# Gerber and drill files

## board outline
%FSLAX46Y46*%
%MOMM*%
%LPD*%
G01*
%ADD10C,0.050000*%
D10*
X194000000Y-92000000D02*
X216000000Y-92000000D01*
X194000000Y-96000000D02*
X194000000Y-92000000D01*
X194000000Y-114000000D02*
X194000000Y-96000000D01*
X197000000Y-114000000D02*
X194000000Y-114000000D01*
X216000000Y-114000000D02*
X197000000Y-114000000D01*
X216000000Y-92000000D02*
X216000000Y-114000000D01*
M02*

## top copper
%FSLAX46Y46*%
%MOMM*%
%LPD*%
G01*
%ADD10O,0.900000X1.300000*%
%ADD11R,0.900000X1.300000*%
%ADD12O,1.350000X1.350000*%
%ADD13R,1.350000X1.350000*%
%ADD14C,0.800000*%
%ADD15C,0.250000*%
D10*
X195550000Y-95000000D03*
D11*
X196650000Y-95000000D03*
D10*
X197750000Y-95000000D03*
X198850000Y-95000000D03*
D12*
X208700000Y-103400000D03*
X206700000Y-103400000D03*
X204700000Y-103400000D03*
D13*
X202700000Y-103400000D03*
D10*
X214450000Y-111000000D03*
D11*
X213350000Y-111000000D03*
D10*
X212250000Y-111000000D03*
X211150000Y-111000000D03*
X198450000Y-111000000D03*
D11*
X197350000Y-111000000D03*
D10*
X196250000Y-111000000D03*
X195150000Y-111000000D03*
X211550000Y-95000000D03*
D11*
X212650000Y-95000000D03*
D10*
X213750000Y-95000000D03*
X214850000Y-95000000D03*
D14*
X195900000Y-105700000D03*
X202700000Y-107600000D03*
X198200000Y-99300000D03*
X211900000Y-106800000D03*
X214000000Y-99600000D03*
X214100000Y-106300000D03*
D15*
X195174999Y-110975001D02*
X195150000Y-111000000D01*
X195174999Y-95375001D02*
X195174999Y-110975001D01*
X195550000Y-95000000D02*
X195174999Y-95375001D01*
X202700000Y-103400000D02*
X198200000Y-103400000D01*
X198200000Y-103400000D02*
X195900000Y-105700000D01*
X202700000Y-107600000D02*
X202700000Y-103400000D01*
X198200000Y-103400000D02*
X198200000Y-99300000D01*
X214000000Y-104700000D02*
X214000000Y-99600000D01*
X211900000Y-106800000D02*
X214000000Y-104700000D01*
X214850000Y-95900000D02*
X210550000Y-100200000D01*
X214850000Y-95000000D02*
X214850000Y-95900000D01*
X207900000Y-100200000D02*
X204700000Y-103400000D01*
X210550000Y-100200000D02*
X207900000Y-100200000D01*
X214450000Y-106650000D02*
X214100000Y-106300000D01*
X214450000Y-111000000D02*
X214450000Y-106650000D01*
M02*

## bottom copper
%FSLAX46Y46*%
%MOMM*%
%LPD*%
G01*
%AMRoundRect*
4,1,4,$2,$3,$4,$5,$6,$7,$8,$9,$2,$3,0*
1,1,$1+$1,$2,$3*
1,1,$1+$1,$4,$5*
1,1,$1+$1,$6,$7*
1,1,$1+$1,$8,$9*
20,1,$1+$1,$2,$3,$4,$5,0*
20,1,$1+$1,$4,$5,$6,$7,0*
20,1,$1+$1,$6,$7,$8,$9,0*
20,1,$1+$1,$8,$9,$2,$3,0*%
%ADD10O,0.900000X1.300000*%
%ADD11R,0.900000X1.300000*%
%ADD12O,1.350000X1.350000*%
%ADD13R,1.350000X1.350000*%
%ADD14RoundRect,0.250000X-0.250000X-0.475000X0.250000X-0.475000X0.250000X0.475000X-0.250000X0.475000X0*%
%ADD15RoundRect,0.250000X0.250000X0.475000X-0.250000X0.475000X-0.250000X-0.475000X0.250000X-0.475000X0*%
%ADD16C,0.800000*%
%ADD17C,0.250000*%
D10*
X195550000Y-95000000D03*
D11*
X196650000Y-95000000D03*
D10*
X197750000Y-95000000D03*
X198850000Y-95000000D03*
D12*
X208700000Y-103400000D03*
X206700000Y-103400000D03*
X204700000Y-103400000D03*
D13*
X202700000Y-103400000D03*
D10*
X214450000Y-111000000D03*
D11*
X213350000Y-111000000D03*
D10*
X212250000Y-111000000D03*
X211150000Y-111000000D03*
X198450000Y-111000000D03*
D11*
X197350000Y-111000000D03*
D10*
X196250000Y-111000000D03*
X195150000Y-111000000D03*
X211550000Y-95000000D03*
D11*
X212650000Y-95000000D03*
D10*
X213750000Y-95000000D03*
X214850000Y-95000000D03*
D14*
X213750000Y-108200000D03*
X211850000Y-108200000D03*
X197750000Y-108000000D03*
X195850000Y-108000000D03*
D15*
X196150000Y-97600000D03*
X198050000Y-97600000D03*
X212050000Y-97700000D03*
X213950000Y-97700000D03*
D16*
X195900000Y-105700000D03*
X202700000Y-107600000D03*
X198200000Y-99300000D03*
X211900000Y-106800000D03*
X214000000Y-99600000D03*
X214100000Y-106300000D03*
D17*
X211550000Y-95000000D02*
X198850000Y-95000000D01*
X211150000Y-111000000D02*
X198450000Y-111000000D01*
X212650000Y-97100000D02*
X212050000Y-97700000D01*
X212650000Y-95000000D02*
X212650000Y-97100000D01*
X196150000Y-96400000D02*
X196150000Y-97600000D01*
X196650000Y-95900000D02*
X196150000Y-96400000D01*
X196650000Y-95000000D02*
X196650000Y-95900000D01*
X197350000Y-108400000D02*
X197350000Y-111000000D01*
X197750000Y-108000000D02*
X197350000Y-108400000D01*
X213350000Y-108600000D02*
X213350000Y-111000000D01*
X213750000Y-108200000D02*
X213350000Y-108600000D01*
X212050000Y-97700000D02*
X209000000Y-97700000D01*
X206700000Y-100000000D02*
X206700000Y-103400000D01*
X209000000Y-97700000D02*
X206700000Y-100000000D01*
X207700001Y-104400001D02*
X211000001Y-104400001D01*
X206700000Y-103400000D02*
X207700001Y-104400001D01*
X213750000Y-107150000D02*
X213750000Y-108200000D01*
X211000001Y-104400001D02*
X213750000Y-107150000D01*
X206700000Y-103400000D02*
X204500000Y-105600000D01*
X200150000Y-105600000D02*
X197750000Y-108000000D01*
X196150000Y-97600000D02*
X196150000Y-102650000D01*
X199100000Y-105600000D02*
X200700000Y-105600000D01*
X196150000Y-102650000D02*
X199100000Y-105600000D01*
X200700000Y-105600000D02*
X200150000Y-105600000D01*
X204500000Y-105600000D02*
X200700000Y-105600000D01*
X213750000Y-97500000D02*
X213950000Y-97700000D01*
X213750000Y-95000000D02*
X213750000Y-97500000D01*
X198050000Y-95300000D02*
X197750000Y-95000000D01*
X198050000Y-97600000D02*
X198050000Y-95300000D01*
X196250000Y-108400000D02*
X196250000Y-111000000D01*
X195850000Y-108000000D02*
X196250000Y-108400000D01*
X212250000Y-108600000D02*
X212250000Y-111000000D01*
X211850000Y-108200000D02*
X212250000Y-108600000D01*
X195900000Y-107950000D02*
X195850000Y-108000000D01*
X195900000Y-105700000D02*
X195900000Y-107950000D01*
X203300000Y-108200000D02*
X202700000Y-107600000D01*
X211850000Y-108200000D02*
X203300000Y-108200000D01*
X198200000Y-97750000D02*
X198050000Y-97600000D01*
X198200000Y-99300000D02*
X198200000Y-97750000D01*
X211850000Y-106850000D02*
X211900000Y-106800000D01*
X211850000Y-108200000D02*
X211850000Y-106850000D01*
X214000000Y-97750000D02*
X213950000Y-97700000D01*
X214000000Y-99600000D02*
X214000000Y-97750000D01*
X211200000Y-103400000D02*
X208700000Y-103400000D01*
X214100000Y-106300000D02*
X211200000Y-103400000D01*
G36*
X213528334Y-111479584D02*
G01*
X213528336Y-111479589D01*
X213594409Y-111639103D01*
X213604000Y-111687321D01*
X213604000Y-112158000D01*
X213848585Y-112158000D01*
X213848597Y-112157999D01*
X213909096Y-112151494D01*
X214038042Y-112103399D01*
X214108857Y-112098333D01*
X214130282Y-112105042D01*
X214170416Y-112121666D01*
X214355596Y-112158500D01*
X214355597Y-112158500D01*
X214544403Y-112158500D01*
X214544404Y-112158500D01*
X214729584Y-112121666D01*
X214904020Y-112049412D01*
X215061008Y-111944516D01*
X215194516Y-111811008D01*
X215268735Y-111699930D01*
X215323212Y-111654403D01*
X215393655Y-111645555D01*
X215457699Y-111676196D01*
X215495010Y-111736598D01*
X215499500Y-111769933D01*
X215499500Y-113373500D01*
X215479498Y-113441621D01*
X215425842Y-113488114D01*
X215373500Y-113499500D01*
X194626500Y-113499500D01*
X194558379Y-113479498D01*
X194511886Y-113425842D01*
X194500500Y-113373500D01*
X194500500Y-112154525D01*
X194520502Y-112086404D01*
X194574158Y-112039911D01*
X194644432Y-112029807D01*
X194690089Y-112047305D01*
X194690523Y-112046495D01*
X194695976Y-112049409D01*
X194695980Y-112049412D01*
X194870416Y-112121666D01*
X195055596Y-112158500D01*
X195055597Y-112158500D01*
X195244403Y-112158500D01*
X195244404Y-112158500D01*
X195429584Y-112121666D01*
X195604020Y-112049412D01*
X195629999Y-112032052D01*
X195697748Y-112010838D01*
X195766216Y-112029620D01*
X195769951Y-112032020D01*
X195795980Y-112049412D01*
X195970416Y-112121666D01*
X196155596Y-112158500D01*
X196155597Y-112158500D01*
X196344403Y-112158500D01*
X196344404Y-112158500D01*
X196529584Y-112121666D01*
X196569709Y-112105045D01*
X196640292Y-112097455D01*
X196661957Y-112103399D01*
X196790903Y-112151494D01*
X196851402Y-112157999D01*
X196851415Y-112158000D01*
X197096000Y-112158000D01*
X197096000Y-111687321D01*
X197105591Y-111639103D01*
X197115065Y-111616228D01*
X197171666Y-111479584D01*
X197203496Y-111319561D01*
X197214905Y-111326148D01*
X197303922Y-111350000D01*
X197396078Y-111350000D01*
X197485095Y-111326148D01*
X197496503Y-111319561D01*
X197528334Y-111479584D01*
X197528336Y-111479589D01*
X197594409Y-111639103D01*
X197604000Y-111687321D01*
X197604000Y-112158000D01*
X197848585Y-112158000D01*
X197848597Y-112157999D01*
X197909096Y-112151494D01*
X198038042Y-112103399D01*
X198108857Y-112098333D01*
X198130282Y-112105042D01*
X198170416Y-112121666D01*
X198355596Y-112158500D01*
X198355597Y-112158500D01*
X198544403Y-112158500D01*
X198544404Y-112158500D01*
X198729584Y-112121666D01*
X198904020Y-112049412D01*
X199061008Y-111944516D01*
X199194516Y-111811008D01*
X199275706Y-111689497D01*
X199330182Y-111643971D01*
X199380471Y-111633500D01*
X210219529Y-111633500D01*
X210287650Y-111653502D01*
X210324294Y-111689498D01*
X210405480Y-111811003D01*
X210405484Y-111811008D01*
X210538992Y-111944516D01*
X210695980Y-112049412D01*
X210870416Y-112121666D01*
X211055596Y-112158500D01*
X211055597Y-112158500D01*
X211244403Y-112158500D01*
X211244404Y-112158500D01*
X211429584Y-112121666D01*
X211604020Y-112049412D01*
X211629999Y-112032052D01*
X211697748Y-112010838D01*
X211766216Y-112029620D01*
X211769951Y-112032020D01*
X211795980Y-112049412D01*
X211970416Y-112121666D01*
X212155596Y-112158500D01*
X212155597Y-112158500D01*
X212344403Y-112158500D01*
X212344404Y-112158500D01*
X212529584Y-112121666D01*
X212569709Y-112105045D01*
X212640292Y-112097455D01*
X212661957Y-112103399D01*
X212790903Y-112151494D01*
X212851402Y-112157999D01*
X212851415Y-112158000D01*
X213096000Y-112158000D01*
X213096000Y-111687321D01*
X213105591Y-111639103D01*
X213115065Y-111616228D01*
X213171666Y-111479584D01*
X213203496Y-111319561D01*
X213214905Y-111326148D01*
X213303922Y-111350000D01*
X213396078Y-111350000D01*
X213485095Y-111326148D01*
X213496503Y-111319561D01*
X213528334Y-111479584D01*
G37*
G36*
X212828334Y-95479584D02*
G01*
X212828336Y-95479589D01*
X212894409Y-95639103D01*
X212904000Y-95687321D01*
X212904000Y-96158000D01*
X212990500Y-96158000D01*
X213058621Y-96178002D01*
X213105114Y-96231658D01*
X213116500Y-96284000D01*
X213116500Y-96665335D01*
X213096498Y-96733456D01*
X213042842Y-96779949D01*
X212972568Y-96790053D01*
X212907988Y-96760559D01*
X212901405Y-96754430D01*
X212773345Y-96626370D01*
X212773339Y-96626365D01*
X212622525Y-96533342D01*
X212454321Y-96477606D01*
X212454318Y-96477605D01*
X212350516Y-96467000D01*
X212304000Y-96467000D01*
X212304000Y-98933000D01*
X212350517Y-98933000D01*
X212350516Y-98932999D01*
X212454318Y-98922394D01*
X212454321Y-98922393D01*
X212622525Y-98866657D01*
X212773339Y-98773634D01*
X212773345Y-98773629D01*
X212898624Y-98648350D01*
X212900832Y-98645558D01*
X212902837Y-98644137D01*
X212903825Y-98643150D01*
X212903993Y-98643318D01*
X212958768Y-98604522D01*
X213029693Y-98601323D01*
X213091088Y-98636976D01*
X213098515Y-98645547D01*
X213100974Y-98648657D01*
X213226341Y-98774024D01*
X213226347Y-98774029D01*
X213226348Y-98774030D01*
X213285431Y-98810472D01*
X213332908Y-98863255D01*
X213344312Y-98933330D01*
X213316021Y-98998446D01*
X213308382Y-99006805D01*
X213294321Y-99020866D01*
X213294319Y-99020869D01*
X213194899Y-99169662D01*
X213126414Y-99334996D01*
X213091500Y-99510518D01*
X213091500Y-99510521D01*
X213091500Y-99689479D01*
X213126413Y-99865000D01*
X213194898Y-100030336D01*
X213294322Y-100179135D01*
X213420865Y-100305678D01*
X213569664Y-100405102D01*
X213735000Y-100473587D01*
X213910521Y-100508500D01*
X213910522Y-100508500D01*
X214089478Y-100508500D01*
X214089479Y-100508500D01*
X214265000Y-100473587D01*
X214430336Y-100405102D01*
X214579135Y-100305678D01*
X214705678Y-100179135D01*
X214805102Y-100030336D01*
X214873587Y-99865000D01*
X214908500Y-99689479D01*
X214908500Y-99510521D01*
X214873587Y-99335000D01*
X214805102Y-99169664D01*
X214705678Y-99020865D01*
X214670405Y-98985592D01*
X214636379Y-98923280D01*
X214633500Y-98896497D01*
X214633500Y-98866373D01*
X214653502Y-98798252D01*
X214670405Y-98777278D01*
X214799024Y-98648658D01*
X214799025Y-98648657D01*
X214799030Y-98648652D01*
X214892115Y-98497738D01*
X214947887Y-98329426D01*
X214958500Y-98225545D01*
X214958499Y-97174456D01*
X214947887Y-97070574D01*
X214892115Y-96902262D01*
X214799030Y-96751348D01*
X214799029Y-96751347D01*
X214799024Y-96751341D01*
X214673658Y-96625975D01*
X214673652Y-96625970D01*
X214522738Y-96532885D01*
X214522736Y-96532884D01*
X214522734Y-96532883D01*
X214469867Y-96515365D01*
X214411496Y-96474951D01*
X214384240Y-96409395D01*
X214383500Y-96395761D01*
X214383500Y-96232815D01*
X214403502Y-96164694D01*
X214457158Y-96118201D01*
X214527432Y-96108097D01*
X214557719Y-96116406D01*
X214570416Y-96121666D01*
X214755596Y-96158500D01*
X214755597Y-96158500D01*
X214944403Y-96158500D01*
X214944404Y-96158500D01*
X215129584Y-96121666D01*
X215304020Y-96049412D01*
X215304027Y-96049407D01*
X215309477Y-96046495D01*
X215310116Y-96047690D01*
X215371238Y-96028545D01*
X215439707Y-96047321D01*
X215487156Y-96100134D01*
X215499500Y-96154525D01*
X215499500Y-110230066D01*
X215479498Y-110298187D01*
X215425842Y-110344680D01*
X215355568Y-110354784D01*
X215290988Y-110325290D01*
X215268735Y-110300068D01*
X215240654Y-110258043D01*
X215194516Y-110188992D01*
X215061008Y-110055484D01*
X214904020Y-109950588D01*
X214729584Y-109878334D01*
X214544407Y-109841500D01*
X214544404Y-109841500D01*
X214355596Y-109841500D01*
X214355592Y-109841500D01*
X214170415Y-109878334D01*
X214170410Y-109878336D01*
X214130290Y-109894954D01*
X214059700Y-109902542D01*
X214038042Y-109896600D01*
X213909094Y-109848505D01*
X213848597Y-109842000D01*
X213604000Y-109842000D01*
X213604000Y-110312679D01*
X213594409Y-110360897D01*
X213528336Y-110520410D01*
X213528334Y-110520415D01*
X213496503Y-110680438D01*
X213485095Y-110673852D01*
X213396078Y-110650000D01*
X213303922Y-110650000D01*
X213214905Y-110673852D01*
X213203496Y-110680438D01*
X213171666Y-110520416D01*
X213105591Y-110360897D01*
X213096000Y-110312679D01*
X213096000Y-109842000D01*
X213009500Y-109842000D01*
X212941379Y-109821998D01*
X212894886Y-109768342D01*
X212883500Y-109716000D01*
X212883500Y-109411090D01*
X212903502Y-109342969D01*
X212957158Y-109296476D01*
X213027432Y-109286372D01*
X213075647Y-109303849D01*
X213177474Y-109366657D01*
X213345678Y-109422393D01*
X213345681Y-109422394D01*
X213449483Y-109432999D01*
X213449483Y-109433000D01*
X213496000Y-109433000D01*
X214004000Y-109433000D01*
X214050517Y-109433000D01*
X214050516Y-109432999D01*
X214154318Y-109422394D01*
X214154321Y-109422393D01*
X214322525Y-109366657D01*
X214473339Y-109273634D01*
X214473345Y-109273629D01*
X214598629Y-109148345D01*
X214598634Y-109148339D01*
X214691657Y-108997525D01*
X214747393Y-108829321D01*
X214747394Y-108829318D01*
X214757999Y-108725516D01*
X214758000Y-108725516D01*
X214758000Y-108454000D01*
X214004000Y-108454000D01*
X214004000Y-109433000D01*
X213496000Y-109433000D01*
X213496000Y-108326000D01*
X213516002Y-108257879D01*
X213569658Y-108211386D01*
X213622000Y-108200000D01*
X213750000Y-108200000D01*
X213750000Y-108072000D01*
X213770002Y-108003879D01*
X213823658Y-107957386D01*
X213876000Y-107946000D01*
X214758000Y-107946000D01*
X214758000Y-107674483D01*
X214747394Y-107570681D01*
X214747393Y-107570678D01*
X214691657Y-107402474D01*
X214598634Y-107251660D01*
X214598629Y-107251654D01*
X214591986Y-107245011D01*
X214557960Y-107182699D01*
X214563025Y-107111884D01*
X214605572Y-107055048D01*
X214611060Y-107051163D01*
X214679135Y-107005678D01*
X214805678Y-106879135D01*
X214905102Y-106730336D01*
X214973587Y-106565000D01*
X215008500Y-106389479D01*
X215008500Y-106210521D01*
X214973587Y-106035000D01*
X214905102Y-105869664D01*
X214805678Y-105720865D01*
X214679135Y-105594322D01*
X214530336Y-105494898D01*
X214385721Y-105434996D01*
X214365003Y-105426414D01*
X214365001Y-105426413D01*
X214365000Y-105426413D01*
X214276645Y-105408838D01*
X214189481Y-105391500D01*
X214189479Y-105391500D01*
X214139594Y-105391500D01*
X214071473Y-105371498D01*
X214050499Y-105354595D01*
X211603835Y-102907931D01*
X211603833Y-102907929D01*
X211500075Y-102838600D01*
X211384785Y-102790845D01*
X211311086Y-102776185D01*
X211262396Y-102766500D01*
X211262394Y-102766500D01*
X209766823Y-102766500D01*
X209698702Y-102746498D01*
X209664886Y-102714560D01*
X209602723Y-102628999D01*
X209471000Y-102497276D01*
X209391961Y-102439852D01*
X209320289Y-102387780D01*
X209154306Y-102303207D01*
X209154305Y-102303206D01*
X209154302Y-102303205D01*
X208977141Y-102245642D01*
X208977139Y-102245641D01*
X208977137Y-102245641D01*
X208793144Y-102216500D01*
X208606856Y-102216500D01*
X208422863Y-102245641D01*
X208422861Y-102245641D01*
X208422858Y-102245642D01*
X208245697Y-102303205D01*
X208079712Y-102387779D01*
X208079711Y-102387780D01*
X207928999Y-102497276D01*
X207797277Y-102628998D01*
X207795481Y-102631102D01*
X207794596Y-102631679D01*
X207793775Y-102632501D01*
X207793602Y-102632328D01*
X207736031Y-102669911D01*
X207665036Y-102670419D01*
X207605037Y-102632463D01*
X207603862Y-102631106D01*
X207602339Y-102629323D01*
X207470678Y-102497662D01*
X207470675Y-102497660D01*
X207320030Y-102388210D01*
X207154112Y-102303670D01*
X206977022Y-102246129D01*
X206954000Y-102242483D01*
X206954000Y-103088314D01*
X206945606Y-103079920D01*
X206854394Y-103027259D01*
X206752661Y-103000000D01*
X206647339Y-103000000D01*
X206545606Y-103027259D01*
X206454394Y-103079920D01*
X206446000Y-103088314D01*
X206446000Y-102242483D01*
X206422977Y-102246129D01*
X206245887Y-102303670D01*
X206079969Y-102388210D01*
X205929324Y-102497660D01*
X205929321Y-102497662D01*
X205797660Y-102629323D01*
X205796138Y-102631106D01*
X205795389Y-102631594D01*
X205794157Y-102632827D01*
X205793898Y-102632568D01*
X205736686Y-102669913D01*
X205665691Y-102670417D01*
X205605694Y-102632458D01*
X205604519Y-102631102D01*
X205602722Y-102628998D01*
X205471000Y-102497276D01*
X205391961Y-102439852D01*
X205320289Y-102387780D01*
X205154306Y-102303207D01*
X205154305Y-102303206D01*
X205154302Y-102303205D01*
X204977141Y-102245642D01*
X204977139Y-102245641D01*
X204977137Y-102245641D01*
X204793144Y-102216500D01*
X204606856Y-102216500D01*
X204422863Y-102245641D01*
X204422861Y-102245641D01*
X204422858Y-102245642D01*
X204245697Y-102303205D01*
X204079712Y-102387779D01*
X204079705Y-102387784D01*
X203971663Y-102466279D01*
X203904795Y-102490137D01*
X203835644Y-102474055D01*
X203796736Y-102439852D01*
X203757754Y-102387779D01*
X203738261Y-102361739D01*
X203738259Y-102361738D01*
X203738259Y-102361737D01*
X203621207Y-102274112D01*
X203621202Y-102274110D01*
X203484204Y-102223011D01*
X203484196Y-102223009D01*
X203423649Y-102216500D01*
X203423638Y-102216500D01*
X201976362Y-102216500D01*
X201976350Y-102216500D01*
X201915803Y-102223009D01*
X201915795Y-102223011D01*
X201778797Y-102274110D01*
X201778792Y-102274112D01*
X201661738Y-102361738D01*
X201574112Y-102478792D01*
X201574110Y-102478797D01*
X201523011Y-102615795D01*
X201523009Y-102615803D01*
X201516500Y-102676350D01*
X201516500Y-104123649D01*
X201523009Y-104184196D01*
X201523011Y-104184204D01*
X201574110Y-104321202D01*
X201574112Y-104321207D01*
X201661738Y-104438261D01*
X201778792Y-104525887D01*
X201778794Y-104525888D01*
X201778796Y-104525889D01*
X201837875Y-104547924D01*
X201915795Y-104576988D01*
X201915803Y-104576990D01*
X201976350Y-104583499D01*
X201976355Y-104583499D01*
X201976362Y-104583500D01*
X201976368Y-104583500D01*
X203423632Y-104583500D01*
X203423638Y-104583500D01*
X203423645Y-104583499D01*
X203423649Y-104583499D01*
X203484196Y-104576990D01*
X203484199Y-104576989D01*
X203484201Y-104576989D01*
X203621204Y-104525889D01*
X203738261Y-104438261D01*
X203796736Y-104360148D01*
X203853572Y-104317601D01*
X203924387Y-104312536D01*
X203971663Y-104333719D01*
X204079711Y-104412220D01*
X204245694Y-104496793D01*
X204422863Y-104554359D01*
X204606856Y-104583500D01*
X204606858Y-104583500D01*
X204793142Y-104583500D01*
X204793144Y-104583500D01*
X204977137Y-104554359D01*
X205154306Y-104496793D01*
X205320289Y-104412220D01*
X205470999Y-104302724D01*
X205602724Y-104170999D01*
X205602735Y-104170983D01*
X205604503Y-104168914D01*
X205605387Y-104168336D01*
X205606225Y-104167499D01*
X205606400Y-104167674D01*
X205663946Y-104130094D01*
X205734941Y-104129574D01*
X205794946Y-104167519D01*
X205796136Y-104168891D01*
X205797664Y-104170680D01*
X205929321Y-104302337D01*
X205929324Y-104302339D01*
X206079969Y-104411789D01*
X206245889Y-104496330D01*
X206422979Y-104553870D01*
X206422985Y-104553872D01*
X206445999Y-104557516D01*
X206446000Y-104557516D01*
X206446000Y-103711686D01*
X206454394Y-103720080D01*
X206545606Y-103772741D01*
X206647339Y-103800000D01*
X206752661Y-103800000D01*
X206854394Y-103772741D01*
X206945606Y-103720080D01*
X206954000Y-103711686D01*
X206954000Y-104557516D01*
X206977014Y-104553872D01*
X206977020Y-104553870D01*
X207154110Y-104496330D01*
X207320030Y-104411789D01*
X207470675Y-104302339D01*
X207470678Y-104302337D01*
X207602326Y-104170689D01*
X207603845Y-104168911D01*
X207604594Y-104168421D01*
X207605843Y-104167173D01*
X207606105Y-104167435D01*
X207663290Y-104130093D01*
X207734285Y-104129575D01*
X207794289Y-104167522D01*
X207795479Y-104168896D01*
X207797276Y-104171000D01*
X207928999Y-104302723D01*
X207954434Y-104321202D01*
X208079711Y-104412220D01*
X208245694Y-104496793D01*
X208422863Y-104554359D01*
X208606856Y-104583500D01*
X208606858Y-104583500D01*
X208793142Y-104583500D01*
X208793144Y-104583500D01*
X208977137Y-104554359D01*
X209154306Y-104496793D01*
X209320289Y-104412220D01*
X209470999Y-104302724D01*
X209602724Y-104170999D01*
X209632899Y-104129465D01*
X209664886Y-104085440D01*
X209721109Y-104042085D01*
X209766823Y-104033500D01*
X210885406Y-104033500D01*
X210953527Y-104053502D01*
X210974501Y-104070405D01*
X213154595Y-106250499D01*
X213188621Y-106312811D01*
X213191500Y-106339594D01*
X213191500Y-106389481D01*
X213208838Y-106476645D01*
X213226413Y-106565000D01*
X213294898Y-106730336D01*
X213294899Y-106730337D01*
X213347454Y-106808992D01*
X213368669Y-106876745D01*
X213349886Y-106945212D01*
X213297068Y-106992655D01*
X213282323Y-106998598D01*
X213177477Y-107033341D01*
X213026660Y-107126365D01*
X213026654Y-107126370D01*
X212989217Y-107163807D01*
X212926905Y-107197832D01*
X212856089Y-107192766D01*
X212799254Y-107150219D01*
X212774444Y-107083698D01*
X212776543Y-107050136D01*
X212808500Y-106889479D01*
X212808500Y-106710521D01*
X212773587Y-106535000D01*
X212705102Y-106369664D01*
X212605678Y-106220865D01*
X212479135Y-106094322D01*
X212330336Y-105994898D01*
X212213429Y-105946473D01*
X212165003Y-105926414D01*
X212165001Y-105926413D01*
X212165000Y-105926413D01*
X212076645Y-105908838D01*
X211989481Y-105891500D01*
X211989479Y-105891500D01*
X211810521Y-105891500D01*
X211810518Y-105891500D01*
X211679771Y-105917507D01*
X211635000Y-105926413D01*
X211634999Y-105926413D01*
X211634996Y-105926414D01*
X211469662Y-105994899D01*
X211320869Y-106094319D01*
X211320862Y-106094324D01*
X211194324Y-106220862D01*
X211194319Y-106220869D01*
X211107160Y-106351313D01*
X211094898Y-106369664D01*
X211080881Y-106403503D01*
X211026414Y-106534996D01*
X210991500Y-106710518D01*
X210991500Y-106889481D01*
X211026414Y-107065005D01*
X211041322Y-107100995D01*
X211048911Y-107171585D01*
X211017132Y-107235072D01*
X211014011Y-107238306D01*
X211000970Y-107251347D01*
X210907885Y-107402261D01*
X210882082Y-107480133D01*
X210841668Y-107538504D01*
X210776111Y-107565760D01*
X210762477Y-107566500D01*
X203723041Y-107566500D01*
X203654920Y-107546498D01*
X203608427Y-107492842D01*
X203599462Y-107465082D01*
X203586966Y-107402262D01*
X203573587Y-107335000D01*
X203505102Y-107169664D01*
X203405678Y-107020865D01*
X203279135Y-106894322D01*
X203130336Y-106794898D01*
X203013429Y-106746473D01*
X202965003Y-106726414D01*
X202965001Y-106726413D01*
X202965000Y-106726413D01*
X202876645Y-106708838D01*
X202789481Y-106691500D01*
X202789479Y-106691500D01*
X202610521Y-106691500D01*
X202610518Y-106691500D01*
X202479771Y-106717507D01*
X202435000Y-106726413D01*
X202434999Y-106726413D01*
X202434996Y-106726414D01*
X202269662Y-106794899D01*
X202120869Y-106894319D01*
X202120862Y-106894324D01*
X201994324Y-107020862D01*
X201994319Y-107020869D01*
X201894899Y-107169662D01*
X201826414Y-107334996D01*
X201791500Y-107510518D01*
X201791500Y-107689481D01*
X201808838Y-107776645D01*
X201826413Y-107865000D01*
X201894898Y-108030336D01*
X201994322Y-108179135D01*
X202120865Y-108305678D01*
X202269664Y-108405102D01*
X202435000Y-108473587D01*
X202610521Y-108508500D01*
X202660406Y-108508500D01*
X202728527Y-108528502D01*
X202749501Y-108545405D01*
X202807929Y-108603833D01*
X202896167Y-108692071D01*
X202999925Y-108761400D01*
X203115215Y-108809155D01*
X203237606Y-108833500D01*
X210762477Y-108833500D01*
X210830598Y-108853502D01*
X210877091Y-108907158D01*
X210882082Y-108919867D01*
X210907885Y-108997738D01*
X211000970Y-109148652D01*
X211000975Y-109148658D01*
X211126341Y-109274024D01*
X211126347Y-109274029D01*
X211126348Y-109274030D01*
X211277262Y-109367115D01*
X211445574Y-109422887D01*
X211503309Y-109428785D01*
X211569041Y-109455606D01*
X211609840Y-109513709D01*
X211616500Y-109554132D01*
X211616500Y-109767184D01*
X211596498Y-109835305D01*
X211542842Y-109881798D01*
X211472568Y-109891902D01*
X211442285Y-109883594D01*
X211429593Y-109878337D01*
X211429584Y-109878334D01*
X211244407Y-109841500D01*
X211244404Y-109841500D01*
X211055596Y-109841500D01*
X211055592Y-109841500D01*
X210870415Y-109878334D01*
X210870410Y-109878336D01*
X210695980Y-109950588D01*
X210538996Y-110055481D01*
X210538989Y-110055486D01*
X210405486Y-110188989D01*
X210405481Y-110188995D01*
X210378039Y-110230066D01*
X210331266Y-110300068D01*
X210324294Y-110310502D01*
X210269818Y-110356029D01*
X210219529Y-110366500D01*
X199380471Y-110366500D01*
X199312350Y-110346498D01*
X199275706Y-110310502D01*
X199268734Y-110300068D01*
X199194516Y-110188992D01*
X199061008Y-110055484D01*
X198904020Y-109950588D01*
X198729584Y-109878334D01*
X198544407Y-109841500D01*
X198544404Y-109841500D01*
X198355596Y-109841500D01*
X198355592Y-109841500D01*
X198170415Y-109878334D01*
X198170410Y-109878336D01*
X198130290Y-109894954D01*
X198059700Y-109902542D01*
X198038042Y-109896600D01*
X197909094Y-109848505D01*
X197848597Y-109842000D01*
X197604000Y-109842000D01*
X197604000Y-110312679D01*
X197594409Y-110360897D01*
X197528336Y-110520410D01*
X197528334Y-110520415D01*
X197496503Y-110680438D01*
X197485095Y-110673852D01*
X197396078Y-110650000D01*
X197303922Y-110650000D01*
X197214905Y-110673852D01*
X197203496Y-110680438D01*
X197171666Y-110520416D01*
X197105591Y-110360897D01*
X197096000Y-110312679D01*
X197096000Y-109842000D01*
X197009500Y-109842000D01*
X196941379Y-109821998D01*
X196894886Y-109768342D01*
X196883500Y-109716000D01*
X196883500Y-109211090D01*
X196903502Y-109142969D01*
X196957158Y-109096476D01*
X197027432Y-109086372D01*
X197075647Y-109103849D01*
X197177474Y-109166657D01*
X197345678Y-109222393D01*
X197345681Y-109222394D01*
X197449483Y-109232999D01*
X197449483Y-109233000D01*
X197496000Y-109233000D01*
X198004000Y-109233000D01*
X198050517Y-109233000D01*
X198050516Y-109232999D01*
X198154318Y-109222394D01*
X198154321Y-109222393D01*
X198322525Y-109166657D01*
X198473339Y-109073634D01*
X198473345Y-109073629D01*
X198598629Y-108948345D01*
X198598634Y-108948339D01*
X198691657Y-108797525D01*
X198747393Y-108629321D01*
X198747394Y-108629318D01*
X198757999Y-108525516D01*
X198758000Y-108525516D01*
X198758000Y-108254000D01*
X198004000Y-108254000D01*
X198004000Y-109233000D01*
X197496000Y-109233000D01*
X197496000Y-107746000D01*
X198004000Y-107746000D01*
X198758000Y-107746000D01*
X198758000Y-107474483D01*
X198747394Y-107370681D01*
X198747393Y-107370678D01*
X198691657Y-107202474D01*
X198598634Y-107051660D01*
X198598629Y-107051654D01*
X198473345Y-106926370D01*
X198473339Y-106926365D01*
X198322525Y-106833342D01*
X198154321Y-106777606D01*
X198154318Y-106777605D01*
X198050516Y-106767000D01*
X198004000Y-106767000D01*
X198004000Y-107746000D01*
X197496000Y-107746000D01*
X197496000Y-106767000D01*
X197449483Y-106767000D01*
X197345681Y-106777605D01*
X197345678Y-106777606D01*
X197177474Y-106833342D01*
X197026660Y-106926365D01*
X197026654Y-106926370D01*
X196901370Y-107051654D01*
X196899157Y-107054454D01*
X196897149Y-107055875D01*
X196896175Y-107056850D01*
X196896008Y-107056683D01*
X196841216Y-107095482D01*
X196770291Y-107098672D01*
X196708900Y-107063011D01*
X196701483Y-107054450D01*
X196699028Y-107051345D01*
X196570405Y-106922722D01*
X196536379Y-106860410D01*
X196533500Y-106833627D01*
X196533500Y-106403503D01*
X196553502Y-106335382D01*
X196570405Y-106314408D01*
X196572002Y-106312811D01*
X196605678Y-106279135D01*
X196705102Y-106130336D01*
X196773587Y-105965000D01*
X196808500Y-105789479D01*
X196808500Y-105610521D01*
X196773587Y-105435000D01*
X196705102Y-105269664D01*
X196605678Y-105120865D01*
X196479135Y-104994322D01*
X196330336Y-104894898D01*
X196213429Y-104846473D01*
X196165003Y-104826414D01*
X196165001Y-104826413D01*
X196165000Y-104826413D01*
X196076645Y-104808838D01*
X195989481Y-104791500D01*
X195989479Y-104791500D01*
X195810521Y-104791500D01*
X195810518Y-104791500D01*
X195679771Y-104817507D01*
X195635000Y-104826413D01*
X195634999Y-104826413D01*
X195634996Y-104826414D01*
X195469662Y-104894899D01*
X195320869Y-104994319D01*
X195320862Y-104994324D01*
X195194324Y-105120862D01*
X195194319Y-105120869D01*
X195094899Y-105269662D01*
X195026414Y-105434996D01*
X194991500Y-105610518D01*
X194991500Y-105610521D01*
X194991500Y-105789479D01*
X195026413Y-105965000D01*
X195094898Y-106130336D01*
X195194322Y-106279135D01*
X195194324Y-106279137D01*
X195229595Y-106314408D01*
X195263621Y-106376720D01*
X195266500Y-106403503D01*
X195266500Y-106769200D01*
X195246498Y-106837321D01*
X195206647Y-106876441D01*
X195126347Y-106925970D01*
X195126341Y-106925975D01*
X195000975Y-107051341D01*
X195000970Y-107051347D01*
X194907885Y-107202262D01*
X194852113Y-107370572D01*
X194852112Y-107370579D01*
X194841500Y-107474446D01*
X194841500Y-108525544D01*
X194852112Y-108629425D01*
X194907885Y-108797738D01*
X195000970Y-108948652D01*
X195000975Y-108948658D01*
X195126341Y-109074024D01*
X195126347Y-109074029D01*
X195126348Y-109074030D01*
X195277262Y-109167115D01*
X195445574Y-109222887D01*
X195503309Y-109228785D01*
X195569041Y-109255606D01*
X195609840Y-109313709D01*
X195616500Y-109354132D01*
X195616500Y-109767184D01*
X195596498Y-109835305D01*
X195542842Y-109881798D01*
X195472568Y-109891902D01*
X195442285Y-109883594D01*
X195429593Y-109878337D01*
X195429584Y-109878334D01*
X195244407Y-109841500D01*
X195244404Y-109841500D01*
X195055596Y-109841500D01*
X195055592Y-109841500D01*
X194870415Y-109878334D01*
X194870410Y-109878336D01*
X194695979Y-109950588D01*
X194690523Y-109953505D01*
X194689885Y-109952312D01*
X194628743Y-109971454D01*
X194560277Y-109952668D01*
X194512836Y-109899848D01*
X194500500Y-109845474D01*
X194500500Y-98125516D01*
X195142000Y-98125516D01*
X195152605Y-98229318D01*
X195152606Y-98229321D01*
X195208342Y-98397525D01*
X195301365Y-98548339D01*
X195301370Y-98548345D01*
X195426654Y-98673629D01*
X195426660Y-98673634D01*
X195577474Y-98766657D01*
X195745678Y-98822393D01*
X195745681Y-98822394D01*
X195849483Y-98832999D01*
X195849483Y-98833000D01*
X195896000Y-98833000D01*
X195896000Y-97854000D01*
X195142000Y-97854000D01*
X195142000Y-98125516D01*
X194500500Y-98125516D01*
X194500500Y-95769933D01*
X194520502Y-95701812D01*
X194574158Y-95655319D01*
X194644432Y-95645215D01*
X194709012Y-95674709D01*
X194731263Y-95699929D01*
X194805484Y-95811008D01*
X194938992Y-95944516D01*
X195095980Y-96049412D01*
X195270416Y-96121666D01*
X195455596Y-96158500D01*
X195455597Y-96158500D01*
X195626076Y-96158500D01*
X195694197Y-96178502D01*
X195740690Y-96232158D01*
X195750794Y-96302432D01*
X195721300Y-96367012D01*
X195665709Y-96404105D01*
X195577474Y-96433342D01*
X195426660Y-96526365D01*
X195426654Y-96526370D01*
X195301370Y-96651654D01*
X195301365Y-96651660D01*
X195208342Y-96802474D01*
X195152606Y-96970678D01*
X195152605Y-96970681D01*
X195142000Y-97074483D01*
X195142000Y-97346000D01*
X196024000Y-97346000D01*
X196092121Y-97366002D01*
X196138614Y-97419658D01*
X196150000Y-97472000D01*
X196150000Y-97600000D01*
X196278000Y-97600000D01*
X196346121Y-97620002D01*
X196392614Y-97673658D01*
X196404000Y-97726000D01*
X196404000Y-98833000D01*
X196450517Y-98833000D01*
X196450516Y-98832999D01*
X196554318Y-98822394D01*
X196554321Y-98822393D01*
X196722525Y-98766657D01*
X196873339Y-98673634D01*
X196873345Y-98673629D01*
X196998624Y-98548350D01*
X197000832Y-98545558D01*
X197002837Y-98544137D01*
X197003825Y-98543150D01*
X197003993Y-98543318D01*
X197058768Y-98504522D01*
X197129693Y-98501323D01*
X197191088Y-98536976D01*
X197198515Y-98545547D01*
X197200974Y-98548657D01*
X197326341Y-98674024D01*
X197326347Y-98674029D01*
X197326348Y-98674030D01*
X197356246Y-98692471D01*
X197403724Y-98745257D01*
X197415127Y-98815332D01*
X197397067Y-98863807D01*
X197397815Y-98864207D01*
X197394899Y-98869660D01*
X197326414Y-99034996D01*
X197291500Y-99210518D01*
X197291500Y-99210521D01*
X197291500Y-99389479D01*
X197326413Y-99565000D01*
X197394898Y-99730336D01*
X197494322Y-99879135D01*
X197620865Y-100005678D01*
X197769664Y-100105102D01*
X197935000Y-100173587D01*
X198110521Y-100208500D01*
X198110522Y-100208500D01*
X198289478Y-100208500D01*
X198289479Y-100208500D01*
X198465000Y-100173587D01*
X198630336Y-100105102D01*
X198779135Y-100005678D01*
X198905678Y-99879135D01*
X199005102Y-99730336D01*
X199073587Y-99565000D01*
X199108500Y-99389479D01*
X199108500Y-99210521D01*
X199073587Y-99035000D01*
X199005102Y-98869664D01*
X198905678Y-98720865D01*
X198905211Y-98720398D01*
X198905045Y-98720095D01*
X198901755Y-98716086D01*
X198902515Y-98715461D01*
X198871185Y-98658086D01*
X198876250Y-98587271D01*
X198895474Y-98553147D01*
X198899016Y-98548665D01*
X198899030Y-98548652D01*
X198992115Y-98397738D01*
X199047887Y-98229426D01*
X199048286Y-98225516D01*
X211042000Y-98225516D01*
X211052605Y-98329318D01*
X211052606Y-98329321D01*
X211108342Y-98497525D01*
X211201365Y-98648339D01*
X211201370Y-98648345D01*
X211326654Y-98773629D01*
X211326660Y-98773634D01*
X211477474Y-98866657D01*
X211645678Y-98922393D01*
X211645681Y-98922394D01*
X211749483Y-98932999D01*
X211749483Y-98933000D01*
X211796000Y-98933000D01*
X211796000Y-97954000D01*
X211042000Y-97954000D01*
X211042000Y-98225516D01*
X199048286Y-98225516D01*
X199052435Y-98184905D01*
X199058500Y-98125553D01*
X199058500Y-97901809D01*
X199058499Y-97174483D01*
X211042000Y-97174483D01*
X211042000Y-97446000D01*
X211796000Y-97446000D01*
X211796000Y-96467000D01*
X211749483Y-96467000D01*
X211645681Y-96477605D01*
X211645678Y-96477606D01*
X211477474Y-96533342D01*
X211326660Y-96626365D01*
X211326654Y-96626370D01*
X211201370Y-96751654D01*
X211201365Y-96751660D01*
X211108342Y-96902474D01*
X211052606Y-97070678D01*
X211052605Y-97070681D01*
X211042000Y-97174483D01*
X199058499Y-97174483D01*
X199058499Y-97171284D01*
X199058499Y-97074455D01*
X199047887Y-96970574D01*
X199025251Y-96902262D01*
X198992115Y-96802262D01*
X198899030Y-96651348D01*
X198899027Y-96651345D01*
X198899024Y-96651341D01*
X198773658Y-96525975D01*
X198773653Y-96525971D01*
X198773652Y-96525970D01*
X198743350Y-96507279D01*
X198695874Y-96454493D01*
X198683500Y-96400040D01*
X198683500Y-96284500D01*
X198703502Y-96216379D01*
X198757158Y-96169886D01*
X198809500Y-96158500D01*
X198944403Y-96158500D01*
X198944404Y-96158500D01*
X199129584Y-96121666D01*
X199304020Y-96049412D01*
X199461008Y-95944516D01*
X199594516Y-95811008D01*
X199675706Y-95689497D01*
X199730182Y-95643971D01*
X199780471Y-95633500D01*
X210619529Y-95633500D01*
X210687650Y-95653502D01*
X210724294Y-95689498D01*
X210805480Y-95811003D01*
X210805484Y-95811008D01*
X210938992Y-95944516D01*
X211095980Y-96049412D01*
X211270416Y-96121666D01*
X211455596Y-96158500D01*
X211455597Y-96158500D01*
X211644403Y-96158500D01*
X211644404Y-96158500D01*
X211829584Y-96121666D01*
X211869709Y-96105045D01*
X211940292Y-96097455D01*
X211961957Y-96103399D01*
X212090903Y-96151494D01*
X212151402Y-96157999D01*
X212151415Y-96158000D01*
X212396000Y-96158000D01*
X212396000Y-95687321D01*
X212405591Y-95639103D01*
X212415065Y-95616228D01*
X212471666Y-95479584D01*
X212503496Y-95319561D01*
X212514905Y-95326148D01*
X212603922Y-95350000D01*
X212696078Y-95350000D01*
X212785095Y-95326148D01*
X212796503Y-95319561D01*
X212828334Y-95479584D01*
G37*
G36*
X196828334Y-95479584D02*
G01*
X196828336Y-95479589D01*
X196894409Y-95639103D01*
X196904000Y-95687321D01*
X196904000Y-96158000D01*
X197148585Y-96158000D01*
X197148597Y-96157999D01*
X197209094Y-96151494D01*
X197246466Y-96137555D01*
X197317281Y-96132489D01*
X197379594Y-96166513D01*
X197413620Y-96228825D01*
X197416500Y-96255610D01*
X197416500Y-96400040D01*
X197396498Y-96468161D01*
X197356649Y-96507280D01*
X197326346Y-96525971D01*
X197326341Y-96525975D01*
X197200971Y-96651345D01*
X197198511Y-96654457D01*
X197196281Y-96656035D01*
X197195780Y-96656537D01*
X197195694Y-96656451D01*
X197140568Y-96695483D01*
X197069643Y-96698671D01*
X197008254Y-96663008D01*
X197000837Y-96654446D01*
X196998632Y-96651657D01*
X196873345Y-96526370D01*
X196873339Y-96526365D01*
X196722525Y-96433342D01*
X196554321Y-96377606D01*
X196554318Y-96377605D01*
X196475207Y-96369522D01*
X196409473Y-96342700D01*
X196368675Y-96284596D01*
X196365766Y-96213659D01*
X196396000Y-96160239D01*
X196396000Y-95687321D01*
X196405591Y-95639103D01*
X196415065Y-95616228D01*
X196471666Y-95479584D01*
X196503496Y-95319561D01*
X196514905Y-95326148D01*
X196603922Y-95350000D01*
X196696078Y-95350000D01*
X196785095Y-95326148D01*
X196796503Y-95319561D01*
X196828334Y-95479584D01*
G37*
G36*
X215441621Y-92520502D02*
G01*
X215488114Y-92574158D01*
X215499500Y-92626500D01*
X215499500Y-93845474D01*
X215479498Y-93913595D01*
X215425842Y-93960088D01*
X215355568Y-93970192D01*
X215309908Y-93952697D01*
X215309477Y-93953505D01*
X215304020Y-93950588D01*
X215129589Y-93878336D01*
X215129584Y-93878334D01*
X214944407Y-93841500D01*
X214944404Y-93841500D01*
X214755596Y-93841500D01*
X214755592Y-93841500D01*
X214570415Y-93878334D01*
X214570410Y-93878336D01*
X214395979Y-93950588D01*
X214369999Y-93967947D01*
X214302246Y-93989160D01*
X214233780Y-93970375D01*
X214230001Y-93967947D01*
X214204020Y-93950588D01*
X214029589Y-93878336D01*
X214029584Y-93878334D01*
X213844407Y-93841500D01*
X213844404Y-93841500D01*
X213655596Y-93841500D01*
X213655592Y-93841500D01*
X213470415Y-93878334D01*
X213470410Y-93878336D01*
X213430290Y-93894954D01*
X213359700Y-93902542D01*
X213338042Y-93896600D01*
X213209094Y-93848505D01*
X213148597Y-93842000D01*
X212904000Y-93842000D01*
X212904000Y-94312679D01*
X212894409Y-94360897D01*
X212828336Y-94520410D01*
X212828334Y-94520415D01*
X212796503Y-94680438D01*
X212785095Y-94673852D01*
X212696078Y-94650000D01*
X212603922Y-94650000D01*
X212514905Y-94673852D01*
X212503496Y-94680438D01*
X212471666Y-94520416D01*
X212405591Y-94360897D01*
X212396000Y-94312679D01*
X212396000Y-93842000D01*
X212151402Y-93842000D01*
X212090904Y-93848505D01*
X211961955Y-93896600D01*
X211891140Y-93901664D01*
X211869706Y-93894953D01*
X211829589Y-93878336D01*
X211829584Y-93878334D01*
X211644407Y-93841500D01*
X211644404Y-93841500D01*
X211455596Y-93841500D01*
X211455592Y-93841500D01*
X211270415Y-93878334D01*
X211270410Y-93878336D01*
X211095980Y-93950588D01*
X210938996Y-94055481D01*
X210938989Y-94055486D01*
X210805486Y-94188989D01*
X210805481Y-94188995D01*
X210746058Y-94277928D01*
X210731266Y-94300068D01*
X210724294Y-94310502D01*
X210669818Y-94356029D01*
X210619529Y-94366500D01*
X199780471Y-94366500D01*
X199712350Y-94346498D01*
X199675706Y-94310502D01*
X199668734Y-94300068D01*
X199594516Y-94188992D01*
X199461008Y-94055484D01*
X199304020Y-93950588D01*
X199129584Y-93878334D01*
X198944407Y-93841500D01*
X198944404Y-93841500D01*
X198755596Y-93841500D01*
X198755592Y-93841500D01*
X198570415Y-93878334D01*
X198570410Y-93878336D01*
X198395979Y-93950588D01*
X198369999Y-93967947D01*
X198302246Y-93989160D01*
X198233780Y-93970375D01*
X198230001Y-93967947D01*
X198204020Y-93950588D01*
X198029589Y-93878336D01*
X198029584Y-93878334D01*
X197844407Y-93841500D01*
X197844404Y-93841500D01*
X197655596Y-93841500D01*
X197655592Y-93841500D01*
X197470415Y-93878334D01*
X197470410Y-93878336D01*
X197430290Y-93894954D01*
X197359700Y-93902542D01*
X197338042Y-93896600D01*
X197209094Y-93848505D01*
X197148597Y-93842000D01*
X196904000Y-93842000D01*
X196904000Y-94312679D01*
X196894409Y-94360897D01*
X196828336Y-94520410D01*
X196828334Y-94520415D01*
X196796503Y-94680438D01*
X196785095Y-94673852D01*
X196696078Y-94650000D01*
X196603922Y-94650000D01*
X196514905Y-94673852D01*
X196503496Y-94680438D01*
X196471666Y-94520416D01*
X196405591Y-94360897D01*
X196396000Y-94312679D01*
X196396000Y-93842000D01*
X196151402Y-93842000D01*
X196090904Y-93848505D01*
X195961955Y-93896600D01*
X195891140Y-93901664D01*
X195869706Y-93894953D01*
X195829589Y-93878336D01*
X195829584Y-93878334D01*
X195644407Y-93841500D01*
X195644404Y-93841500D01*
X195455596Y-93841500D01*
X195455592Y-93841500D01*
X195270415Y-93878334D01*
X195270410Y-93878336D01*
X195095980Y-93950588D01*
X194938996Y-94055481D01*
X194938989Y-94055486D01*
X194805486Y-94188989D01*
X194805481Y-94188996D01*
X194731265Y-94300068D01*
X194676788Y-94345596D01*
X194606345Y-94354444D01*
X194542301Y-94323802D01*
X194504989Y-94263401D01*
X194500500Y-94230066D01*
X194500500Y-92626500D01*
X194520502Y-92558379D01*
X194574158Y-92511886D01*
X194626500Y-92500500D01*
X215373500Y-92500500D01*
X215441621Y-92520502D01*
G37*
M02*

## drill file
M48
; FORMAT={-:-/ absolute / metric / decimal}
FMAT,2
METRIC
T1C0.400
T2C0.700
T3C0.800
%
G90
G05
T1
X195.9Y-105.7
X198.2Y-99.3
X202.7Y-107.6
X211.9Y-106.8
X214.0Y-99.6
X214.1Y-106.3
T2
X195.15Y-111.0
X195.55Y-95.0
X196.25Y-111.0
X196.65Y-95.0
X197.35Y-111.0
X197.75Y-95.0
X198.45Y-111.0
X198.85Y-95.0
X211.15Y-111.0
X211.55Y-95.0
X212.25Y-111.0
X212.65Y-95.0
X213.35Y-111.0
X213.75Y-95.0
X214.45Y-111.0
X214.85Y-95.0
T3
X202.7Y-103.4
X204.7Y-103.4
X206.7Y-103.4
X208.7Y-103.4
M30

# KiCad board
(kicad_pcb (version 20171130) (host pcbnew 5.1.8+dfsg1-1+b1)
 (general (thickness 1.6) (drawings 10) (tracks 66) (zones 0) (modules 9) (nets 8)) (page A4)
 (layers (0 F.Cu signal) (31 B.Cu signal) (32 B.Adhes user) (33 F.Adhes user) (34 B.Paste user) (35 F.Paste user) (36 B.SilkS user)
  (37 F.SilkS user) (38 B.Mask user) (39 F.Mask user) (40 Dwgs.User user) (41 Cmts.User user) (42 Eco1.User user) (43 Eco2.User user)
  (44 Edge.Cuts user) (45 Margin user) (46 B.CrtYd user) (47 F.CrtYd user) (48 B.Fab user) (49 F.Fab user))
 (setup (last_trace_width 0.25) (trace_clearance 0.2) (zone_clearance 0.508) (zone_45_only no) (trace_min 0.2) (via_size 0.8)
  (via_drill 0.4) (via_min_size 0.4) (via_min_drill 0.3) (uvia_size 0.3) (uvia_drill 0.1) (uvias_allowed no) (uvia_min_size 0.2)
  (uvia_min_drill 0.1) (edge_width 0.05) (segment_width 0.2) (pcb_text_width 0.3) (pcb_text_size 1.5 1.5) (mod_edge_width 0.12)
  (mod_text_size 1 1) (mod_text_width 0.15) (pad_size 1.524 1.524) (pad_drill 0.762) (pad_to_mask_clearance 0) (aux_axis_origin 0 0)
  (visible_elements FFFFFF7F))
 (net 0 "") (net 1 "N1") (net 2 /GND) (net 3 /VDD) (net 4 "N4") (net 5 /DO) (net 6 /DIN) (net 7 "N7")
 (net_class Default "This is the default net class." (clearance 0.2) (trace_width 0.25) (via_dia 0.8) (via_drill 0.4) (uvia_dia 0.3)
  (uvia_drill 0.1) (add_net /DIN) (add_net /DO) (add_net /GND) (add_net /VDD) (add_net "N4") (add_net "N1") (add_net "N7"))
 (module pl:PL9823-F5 (layer F.Cu) (at 197 95 180)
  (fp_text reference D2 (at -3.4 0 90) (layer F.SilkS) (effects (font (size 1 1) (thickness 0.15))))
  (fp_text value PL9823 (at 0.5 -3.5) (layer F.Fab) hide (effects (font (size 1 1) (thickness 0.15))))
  (pad 2 thru_hole oval (at 1.45 0 180) (size 0.9 1.3) (drill 0.7) (layers *.Cu *.Mask) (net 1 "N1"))
  (pad 1 thru_hole rect (at 0.35 0 180) (size 0.9 1.3) (drill 0.7) (layers *.Cu *.Mask) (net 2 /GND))
  (pad 3 thru_hole oval (at -0.75 0 180) (size 0.9 1.3) (drill 0.7) (layers *.Cu *.Mask) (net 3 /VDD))
  (pad 4 thru_hole oval (at -1.85 0 180) (size 0.9 1.3) (drill 0.7) (layers *.Cu *.Mask) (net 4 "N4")))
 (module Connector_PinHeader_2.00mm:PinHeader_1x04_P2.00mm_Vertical (layer F.Cu) (at 202.7 103.4 90)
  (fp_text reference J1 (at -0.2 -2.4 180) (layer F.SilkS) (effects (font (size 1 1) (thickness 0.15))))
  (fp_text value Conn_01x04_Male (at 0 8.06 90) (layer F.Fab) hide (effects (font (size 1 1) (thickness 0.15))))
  (pad 4 thru_hole oval (at 0 6 90) (size 1.35 1.35) (drill 0.8) (layers *.Cu *.Mask) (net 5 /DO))
  (pad 3 thru_hole oval (at 0 4 90) (size 1.35 1.35) (drill 0.8) (layers *.Cu *.Mask) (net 2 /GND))
  (pad 2 thru_hole oval (at 0 2 90) (size 1.35 1.35) (drill 0.8) (layers *.Cu *.Mask) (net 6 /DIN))
  (pad 1 thru_hole rect (at 0 0 90) (size 1.35 1.35) (drill 0.8) (layers *.Cu *.Mask) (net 3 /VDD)))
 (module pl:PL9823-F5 (layer F.Cu) (at 213 111)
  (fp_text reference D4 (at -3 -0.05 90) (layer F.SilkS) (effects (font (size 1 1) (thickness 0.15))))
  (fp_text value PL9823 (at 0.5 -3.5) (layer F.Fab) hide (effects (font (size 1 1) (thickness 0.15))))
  (pad 2 thru_hole oval (at 1.45 0) (size 0.9 1.3) (drill 0.7) (layers *.Cu *.Mask) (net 5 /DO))
  (pad 1 thru_hole rect (at 0.35 0) (size 0.9 1.3) (drill 0.7) (layers *.Cu *.Mask) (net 2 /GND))
  (pad 3 thru_hole oval (at -0.75 0) (size 0.9 1.3) (drill 0.7) (layers *.Cu *.Mask) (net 3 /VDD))
  (pad 4 thru_hole oval (at -1.85 0) (size 0.9 1.3) (drill 0.7) (layers *.Cu *.Mask) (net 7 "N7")))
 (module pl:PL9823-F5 (layer F.Cu) (at 197 111)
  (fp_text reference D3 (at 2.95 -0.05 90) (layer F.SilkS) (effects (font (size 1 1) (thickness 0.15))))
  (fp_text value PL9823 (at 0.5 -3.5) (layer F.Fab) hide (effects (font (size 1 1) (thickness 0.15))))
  (pad 2 thru_hole oval (at 1.45 0) (size 0.9 1.3) (drill 0.7) (layers *.Cu *.Mask) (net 7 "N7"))
  (pad 1 thru_hole rect (at 0.35 0) (size 0.9 1.3) (drill 0.7) (layers *.Cu *.Mask) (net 2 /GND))
  (pad 3 thru_hole oval (at -0.75 0) (size 0.9 1.3) (drill 0.7) (layers *.Cu *.Mask) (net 3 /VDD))
  (pad 4 thru_hole oval (at -1.85 0) (size 0.9 1.3) (drill 0.7) (layers *.Cu *.Mask) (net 1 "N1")))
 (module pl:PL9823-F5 (layer F.Cu) (at 213 95 180)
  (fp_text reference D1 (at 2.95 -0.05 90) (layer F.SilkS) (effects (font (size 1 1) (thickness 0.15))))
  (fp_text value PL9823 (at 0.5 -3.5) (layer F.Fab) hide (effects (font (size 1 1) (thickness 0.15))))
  (pad 2 thru_hole oval (at 1.45 0 180) (size 0.9 1.3) (drill 0.7) (layers *.Cu *.Mask) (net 4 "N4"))
  (pad 1 thru_hole rect (at 0.35 0 180) (size 0.9 1.3) (drill 0.7) (layers *.Cu *.Mask) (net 2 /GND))
  (pad 3 thru_hole oval (at -0.75 0 180) (size 0.9 1.3) (drill 0.7) (layers *.Cu *.Mask) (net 3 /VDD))
  (pad 4 thru_hole oval (at -1.85 0 180) (size 0.9 1.3) (drill 0.7) (layers *.Cu *.Mask) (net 6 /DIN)))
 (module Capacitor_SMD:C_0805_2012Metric (layer B.Cu) (at 212.8 108.2)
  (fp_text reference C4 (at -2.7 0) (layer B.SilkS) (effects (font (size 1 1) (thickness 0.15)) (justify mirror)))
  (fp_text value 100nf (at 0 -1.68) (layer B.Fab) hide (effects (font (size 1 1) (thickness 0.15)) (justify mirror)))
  (pad 2 smd roundrect (at 0.95 0) (size 1 1.45) (layers B.Cu B.Paste B.Mask) (roundrect_rratio 0.25) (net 2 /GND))
  (pad 1 smd roundrect (at -0.95 0) (size 1 1.45) (layers B.Cu B.Paste B.Mask) (roundrect_rratio 0.25) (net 3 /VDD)))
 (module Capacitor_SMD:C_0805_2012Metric (layer B.Cu) (at 196.8 108)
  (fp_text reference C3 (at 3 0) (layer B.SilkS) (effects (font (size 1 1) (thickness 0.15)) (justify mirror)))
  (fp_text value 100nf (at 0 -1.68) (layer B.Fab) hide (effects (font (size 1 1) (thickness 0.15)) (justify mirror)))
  (pad 2 smd roundrect (at 0.95 0) (size 1 1.45) (layers B.Cu B.Paste B.Mask) (roundrect_rratio 0.25) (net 2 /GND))
  (pad 1 smd roundrect (at -0.95 0) (size 1 1.45) (layers B.Cu B.Paste B.Mask) (roundrect_rratio 0.25) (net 3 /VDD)))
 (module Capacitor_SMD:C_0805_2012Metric (layer B.Cu) (at 197.1 97.6 180)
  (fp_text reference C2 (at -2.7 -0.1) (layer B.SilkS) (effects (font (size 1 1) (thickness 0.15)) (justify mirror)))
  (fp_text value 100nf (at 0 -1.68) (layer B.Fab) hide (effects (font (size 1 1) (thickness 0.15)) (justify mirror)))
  (pad 2 smd roundrect (at 0.95 0 180) (size 1 1.45) (layers B.Cu B.Paste B.Mask) (roundrect_rratio 0.25) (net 2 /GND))
  (pad 1 smd roundrect (at -0.95 0 180) (size 1 1.45) (layers B.Cu B.Paste B.Mask) (roundrect_rratio 0.25) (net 3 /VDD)))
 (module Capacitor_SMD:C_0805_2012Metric (layer B.Cu) (at 213 97.7 180)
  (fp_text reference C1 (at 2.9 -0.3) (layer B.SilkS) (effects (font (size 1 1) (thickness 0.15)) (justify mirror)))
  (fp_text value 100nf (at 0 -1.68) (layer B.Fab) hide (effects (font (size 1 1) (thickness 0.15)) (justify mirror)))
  (pad 2 smd roundrect (at 0.95 0 180) (size 1 1.45) (layers B.Cu B.Paste B.Mask) (roundrect_rratio 0.25) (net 2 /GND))
  (pad 1 smd roundrect (at -0.95 0 180) (size 1 1.45) (layers B.Cu B.Paste B.Mask) (roundrect_rratio 0.25) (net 3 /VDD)))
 (gr_line (start 194 92) (end 216 92) (layer Edge.Cuts) (width 0.05))
 (gr_line (start 194 96) (end 194 92) (layer Edge.Cuts) (width 0.05))
 (gr_line (start 194 114) (end 194 96) (layer Edge.Cuts) (width 0.05))
 (gr_line (start 197 114) (end 194 114) (layer Edge.Cuts) (width 0.05))
 (gr_line (start 216 114) (end 197 114) (layer Edge.Cuts) (width 0.05))
 (gr_line (start 216 92) (end 216 114) (layer Edge.Cuts) (width 0.05))
 (segment (start 211.55 95) (end 198.85 95) (width 0.25) (layer B.Cu) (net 4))
 (segment (start 195.174999 110.975001) (end 195.15 111) (width 0.25) (layer F.Cu) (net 1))
 (segment (start 195.174999 95.375001) (end 195.174999 110.975001) (width 0.25) (layer F.Cu) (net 1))
 (segment (start 195.55 95) (end 195.174999 95.375001) (width 0.25) (layer F.Cu) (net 1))
 (segment (start 211.15 111) (end 198.45 111) (width 0.25) (layer B.Cu) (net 7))
 (segment (start 212.65 97.1) (end 212.05 97.7) (width 0.25) (layer B.Cu) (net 2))
 (segment (start 212.65 95) (end 212.65 97.1) (width 0.25) (layer B.Cu) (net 2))
 (segment (start 196.15 96.4) (end 196.15 97.6) (width 0.25) (layer B.Cu) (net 2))
 (segment (start 196.65 95.9) (end 196.15 96.4) (width 0.25) (layer B.Cu) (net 2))
 (segment (start 196.65 95) (end 196.65 95.9) (width 0.25) (layer B.Cu) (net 2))
 (segment (start 197.35 108.4) (end 197.35 111) (width 0.25) (layer B.Cu) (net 2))
 (segment (start 197.75 108) (end 197.35 108.4) (width 0.25) (layer B.Cu) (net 2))
 (segment (start 213.35 108.6) (end 213.35 111) (width 0.25) (layer B.Cu) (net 2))
 (segment (start 213.75 108.2) (end 213.35 108.6) (width 0.25) (layer B.Cu) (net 2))
 (segment (start 212.05 97.7) (end 209 97.7) (width 0.25) (layer B.Cu) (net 2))
 (segment (start 206.7 100) (end 206.7 103.4) (width 0.25) (layer B.Cu) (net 2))
 (segment (start 209 97.7) (end 206.7 100) (width 0.25) (layer B.Cu) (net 2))
 (segment (start 207.700001 104.400001) (end 211.000001 104.400001) (width 0.25) (layer B.Cu) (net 2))
 (segment (start 206.7 103.4) (end 207.700001 104.400001) (width 0.25) (layer B.Cu) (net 2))
 (segment (start 213.75 107.15) (end 213.75 108.2) (width 0.25) (layer B.Cu) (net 2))
 (segment (start 211.000001 104.400001) (end 213.75 107.15) (width 0.25) (layer B.Cu) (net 2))
 (segment (start 206.7 103.4) (end 204.5 105.6) (width 0.25) (layer B.Cu) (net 2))
 (segment (start 200.15 105.6) (end 197.75 108) (width 0.25) (layer B.Cu) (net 2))
 (segment (start 196.15 97.6) (end 196.15 102.65) (width 0.25) (layer B.Cu) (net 2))
 (segment (start 199.1 105.6) (end 200.7 105.6) (width 0.25) (layer B.Cu) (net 2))
 (segment (start 196.15 102.65) (end 199.1 105.6) (width 0.25) (layer B.Cu) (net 2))
 (segment (start 200.7 105.6) (end 200.15 105.6) (width 0.25) (layer B.Cu) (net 2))
 (segment (start 204.5 105.6) (end 200.7 105.6) (width 0.25) (layer B.Cu) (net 2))
 (segment (start 213.75 97.5) (end 213.95 97.7) (width 0.25) (layer B.Cu) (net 3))
 (segment (start 213.75 95) (end 213.75 97.5) (width 0.25) (layer B.Cu) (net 3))
 (segment (start 198.05 95.3) (end 197.75 95) (width 0.25) (layer B.Cu) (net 3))
 (segment (start 198.05 97.6) (end 198.05 95.3) (width 0.25) (layer B.Cu) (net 3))
 (segment (start 196.25 108.4) (end 196.25 111) (width 0.25) (layer B.Cu) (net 3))
 (segment (start 195.85 108) (end 196.25 108.4) (width 0.25) (layer B.Cu) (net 3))
 (segment (start 212.25 108.6) (end 212.25 111) (width 0.25) (layer B.Cu) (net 3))
 (segment (start 211.85 108.2) (end 212.25 108.6) (width 0.25) (layer B.Cu) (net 3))
 (segment (start 202.7 103.4) (end 198.2 103.4) (width 0.25) (layer F.Cu) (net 3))
 (via (at 195.9 105.7) (size 0.8) (drill 0.4) (layers F.Cu B.Cu) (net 3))
 (segment (start 198.2 103.4) (end 195.9 105.7) (width 0.25) (layer F.Cu) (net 3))
 (segment (start 195.9 107.95) (end 195.85 108) (width 0.25) (layer B.Cu) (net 3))
 (segment (start 195.9 105.7) (end 195.9 107.95) (width 0.25) (layer B.Cu) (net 3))
 (via (at 202.7 107.6) (size 0.8) (drill 0.4) (layers F.Cu B.Cu) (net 3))
 (segment (start 203.3 108.2) (end 202.7 107.6) (width 0.25) (layer B.Cu) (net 3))
 (segment (start 211.85 108.2) (end 203.3 108.2) (width 0.25) (layer B.Cu) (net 3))
 (segment (start 202.7 107.6) (end 202.7 103.4) (width 0.25) (layer F.Cu) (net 3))
 (via (at 198.2 99.3) (size 0.8) (drill 0.4) (layers F.Cu B.Cu) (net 3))
 (segment (start 198.2 103.4) (end 198.2 99.3) (width 0.25) (layer F.Cu) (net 3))
 (segment (start 198.2 97.75) (end 198.05 97.6) (width 0.25) (layer B.Cu) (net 3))
 (segment (start 198.2 99.3) (end 198.2 97.75) (width 0.25) (layer B.Cu) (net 3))
 (via (at 211.9 106.8) (size 0.8) (drill 0.4) (layers F.Cu B.Cu) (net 3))
 (segment (start 211.85 106.85) (end 211.9 106.8) (width 0.25) (layer B.Cu) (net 3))
 (segment (start 211.85 108.2) (end 211.85 106.85) (width 0.25) (layer B.Cu) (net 3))
 (segment (start 214 104.7) (end 214 99.6) (width 0.25) (layer F.Cu) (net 3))
 (via (at 214 99.6) (size 0.8) (drill 0.4) (layers F.Cu B.Cu) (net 3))
 (segment (start 211.9 106.8) (end 214 104.7) (width 0.25) (layer F.Cu) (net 3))
 (segment (start 214 97.75) (end 213.95 97.7) (width 0.25) (layer B.Cu) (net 3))
 (segment (start 214 99.6) (end 214 97.75) (width 0.25) (layer B.Cu) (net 3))
 (segment (start 214.85 95.9) (end 210.55 100.2) (width 0.25) (layer F.Cu) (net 6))
 (segment (start 214.85 95) (end 214.85 95.9) (width 0.25) (layer F.Cu) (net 6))
 (segment (start 207.9 100.2) (end 204.7 103.4) (width 0.25) (layer F.Cu) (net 6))
 (segment (start 210.55 100.2) (end 207.9 100.2) (width 0.25) (layer F.Cu) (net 6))
 (via (at 214.1 106.3) (size 0.8) (drill 0.4) (layers F.Cu B.Cu) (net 5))
 (segment (start 214.45 106.65) (end 214.1 106.3) (width 0.25) (layer F.Cu) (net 5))
 (segment (start 214.45 111) (end 214.45 106.65) (width 0.25) (layer F.Cu) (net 5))
 (segment (start 211.2 103.4) (end 208.7 103.4) (width 0.25) (layer B.Cu) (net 5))
 (segment (start 214.1 106.3) (end 211.2 103.4) (width 0.25) (layer B.Cu) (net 5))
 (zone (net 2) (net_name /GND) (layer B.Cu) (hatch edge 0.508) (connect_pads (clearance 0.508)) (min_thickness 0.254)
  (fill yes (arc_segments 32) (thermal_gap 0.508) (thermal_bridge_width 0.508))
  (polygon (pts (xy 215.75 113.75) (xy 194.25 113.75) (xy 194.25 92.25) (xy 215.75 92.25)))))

